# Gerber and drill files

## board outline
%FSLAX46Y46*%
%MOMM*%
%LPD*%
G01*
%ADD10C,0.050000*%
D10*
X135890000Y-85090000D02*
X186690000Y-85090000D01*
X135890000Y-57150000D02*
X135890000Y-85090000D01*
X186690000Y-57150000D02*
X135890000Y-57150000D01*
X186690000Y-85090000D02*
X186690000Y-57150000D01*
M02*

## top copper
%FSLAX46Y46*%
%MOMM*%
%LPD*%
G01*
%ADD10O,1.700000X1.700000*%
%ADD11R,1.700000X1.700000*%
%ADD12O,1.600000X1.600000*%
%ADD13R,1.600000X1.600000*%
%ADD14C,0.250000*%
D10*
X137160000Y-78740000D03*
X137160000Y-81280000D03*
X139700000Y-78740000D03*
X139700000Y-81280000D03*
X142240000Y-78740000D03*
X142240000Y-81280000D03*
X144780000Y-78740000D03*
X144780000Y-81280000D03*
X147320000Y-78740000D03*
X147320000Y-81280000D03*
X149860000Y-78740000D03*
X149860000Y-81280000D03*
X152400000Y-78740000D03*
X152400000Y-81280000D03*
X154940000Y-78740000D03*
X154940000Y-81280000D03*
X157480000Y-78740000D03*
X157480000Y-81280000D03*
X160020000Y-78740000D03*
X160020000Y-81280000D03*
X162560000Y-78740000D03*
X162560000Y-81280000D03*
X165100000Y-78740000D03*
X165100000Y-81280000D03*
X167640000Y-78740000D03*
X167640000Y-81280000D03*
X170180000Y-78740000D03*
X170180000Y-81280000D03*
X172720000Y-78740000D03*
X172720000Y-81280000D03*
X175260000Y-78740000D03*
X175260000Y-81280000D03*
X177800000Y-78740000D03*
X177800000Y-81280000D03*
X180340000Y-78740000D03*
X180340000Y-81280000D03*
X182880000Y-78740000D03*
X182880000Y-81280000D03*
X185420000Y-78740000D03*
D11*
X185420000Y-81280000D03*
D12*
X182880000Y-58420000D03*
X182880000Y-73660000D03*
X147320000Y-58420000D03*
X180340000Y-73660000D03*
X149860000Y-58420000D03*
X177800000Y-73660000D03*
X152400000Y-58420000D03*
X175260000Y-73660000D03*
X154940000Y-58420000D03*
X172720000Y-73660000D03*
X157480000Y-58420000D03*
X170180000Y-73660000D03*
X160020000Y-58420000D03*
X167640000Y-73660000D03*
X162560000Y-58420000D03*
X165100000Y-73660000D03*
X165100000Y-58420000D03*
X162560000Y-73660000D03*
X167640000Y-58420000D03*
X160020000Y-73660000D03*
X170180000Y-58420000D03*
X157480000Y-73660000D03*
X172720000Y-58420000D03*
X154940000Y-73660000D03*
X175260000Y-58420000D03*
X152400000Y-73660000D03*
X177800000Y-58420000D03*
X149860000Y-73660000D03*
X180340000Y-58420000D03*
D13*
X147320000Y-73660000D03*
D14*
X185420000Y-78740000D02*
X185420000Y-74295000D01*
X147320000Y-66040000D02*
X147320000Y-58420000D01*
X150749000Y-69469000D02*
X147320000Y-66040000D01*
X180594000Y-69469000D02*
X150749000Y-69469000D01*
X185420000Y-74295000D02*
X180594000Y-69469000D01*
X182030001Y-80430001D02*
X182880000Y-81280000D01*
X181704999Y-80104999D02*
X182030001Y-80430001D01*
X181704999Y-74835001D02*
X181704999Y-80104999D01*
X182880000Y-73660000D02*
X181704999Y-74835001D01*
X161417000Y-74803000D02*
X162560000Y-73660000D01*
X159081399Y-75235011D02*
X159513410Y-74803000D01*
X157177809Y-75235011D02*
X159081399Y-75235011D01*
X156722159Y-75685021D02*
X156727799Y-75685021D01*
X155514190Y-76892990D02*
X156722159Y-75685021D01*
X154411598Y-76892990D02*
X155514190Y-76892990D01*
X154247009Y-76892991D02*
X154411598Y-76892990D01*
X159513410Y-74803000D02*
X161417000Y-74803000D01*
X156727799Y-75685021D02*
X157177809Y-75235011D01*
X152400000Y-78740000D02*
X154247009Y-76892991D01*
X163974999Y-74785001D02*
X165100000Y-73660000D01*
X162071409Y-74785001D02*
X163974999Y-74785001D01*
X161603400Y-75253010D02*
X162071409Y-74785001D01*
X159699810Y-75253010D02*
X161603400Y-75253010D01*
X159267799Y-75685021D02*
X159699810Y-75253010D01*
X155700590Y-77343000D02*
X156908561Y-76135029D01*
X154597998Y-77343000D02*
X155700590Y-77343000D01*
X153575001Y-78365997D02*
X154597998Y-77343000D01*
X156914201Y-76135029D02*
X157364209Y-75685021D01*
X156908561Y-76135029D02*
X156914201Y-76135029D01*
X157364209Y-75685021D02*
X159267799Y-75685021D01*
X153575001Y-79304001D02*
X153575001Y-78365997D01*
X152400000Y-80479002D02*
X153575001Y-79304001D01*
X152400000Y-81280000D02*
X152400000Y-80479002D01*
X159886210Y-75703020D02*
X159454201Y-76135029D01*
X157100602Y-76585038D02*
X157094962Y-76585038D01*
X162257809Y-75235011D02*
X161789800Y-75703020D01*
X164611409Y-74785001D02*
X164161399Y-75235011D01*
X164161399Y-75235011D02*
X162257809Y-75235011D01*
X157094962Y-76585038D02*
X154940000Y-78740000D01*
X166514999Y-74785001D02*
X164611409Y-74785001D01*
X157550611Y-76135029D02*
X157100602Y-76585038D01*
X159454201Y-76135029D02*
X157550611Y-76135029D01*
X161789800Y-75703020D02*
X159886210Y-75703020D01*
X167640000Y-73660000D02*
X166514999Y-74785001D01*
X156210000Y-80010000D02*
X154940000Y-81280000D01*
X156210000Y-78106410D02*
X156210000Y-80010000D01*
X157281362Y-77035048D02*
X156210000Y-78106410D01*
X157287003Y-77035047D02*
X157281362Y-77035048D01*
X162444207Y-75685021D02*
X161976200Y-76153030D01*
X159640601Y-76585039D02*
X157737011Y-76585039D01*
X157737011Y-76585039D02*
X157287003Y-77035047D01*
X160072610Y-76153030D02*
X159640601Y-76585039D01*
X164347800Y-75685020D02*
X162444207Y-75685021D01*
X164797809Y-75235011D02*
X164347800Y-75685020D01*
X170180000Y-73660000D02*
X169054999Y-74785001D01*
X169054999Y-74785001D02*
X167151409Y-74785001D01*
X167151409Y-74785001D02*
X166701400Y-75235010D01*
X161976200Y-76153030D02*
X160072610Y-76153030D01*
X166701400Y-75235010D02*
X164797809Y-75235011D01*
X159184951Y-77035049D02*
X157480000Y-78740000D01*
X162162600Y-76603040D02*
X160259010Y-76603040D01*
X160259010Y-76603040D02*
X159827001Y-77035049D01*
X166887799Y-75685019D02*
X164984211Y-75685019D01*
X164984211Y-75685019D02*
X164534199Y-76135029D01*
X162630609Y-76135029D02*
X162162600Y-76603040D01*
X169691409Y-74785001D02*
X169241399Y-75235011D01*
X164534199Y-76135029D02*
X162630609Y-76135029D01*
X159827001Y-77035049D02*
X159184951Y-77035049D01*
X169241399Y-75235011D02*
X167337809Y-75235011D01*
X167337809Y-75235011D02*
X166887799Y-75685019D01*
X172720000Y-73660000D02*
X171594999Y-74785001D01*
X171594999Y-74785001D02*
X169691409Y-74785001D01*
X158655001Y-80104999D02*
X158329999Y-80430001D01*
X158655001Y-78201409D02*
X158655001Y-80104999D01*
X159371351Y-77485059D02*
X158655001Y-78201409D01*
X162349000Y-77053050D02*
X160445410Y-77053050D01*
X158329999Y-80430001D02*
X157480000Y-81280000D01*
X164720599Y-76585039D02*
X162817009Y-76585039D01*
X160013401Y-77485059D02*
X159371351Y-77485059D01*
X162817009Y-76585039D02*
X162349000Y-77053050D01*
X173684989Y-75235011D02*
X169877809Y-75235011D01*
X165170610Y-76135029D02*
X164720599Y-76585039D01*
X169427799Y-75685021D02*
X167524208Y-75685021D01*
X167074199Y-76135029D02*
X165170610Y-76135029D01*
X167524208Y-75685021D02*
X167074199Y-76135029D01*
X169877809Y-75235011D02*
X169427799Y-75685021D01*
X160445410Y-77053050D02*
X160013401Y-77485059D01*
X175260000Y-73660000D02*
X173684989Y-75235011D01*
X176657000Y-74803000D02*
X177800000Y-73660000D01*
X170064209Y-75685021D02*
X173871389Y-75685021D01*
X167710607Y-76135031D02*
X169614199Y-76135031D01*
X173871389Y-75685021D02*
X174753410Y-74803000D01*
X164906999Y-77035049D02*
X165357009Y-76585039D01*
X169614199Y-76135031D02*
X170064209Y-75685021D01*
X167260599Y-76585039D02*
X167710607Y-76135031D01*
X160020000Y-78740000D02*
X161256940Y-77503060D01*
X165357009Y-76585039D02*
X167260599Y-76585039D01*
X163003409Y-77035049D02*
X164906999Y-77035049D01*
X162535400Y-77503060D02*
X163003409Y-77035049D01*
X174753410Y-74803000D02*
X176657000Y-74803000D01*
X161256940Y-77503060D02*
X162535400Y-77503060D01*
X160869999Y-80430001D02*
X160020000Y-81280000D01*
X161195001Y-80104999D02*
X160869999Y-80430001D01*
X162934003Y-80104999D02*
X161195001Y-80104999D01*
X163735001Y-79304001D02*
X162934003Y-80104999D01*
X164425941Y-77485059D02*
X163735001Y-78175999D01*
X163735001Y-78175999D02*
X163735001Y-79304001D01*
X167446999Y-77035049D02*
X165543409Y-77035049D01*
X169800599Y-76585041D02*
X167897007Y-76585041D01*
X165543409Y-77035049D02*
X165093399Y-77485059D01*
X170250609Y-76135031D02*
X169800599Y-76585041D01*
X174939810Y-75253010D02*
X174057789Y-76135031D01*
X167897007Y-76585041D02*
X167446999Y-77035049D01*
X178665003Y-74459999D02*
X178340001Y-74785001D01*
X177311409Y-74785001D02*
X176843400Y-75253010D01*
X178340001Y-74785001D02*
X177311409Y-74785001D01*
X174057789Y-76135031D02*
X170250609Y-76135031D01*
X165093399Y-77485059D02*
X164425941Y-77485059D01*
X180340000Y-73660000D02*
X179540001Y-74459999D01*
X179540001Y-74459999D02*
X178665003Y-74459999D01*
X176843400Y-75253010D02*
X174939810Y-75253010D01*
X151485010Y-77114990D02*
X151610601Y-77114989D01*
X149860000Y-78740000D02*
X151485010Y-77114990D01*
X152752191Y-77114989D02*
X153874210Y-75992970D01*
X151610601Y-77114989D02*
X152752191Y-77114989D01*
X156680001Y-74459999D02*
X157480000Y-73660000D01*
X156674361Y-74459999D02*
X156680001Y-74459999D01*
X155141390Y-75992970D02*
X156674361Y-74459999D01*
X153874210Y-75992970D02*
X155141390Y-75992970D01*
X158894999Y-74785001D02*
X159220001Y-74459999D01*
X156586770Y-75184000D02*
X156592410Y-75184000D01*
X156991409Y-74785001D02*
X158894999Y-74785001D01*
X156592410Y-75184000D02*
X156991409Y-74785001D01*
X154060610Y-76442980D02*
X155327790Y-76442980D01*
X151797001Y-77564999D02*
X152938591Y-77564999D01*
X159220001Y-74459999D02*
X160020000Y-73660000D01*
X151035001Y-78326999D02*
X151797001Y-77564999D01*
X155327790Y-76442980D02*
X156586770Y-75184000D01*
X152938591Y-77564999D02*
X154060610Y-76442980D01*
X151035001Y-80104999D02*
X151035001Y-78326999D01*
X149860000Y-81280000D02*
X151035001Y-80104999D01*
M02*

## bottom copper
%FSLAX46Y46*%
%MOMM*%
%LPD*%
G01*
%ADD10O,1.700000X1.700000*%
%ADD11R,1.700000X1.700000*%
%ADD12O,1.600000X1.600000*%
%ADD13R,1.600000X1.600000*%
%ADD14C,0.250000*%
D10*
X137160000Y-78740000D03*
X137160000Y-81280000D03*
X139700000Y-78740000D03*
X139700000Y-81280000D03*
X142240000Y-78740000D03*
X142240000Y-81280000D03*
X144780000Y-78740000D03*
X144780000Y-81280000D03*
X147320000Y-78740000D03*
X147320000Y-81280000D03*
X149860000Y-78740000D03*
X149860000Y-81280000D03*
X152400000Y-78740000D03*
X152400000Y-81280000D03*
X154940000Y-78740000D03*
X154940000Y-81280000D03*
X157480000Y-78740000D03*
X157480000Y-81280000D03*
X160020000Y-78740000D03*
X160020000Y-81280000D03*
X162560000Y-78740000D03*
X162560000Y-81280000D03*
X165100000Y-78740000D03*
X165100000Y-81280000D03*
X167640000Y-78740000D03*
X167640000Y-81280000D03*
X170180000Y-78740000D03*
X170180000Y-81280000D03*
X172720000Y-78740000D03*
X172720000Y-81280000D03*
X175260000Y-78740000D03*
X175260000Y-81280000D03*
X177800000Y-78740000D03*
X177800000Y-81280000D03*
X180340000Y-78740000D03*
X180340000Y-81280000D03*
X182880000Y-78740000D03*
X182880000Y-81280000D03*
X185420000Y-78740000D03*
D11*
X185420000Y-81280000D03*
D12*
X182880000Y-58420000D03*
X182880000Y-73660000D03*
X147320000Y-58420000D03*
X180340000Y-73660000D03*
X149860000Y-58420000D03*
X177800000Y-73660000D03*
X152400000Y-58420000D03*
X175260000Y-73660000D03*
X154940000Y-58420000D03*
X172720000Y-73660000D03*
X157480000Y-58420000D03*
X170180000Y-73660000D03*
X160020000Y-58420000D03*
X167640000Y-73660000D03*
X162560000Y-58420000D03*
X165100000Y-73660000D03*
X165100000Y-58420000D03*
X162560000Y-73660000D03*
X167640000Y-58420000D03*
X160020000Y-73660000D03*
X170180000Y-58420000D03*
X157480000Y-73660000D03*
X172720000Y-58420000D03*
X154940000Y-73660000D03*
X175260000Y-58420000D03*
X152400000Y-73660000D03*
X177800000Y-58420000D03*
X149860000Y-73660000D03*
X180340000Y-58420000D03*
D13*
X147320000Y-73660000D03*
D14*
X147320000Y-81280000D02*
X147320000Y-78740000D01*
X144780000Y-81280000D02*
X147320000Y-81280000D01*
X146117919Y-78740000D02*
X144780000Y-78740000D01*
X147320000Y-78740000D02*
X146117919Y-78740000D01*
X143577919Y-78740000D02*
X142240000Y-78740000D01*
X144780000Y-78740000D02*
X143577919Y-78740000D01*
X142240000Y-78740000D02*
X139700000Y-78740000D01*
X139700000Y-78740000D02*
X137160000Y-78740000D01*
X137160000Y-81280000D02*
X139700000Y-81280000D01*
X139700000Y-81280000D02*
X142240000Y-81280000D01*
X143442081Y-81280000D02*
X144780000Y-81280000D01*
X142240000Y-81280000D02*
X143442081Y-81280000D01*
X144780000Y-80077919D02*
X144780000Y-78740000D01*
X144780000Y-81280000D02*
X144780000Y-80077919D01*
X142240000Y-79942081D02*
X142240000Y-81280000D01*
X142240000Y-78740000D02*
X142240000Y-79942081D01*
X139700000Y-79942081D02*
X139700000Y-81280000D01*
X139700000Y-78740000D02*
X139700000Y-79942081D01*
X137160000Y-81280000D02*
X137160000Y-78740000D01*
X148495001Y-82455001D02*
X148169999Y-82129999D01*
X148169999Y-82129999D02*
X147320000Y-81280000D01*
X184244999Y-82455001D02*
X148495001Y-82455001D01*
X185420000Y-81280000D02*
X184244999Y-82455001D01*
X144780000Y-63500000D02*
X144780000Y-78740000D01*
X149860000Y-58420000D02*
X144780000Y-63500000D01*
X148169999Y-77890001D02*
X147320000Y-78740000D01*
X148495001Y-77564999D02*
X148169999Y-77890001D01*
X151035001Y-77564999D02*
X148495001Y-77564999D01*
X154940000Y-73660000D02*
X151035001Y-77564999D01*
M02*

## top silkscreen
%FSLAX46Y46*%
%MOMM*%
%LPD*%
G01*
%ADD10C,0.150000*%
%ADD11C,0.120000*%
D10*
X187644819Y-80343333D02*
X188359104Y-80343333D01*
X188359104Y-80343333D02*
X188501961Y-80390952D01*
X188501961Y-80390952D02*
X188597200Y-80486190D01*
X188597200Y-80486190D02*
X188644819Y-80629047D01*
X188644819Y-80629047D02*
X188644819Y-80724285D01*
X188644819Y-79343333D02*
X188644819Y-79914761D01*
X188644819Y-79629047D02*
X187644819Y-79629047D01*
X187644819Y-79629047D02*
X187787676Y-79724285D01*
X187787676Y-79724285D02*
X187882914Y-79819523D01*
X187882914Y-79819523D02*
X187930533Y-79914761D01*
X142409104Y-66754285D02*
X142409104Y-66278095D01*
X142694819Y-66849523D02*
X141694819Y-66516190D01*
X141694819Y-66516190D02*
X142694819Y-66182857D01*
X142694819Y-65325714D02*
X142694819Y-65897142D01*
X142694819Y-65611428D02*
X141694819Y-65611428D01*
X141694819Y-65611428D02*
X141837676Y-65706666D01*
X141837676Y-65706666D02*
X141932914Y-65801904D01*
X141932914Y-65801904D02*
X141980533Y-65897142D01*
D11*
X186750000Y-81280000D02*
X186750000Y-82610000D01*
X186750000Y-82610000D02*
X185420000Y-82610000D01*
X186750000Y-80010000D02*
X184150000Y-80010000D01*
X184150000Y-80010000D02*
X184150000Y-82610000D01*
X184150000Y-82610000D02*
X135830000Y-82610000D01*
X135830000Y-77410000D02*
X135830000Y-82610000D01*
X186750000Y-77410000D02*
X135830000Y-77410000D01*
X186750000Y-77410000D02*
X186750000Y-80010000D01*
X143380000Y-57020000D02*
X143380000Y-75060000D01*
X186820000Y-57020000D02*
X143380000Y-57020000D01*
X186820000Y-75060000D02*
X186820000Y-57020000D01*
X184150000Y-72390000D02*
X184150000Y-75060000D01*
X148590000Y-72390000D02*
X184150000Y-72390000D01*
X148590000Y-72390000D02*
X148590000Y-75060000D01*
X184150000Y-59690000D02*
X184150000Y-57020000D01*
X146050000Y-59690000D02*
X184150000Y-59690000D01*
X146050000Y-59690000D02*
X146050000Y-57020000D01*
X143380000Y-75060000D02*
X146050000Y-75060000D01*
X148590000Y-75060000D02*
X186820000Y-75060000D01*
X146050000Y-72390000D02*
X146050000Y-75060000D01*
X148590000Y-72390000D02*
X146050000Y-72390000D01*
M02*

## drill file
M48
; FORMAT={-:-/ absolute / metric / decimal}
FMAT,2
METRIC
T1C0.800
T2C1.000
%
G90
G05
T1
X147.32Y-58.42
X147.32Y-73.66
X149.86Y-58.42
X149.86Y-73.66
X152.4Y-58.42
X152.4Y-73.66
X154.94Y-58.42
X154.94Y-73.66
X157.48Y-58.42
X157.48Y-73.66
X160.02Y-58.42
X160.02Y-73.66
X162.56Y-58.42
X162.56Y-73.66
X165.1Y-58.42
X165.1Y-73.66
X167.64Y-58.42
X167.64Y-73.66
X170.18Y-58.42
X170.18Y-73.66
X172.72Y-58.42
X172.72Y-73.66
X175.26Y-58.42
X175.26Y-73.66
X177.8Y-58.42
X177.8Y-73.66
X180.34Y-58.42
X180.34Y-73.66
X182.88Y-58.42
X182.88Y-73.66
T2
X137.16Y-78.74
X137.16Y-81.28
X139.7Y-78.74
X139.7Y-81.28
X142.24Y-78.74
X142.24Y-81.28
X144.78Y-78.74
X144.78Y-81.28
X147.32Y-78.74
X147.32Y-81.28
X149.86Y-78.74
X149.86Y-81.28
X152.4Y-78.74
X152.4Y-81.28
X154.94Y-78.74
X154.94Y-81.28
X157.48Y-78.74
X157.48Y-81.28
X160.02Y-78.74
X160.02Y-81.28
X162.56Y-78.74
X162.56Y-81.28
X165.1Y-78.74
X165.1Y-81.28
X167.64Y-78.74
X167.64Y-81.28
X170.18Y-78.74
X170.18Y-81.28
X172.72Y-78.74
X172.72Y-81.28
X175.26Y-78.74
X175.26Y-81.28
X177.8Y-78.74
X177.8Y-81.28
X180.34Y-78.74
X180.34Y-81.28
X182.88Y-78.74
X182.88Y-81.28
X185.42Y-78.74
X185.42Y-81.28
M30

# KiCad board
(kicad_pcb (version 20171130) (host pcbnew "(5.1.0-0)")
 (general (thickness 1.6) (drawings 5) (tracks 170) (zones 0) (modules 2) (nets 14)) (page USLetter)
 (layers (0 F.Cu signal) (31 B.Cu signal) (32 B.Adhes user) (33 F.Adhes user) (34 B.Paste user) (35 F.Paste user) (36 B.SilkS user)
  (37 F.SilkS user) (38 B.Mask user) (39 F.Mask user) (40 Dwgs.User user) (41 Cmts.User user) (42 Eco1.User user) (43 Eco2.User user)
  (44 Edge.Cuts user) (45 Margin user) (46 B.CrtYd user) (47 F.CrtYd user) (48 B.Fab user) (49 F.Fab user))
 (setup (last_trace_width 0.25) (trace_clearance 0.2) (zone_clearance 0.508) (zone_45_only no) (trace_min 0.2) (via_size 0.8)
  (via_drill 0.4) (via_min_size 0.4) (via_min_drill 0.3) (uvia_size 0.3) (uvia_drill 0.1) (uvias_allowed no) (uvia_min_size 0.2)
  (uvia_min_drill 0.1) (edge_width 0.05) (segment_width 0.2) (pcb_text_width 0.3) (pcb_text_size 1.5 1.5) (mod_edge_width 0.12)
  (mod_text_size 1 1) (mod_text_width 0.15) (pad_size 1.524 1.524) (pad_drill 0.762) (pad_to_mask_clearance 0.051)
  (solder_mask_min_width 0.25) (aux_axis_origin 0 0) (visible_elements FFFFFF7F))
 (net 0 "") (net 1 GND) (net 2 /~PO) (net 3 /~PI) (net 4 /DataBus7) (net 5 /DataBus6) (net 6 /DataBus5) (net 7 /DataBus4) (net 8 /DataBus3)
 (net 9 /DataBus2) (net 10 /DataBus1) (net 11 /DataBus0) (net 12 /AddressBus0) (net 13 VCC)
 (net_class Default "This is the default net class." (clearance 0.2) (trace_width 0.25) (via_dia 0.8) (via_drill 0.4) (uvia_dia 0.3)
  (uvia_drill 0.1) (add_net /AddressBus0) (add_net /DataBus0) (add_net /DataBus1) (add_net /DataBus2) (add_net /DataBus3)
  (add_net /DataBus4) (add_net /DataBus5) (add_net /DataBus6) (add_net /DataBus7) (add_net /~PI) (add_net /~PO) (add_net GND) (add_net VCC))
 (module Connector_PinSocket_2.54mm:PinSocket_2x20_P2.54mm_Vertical (layer F.Cu) (at 185.42 81.28 270)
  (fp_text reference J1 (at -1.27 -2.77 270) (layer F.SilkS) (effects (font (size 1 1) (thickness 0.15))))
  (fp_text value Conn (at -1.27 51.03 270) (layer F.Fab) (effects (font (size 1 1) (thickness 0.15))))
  (fp_line (start 0 -1.33) (end 1.33 -1.33) (layer F.SilkS) (width 0.12))
  (fp_line (start 1.33 -1.33) (end 1.33 0) (layer F.SilkS) (width 0.12))
  (fp_line (start -1.27 -1.33) (end -1.27 1.27) (layer F.SilkS) (width 0.12))
  (fp_line (start -1.27 1.27) (end 1.33 1.27) (layer F.SilkS) (width 0.12))
  (fp_line (start 1.33 1.27) (end 1.33 49.59) (layer F.SilkS) (width 0.12))
  (fp_line (start -3.87 49.59) (end 1.33 49.59) (layer F.SilkS) (width 0.12))
  (fp_line (start -3.87 -1.33) (end -3.87 49.59) (layer F.SilkS) (width 0.12))
  (fp_line (start -3.87 -1.33) (end -1.27 -1.33) (layer F.SilkS) (width 0.12))
  (pad 40 thru_hole oval (at -2.54 48.26 270) (size 1.7 1.7) (drill 1) (layers *.Cu *.Mask) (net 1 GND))
  (pad 39 thru_hole oval (at 0 48.26 270) (size 1.7 1.7) (drill 1) (layers *.Cu *.Mask) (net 1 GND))
  (pad 38 thru_hole oval (at -2.54 45.72 270) (size 1.7 1.7) (drill 1) (layers *.Cu *.Mask) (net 1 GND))
  (pad 37 thru_hole oval (at 0 45.72 270) (size 1.7 1.7) (drill 1) (layers *.Cu *.Mask) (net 1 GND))
  (pad 36 thru_hole oval (at -2.54 43.18 270) (size 1.7 1.7) (drill 1) (layers *.Cu *.Mask) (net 1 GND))
  (pad 35 thru_hole oval (at 0 43.18 270) (size 1.7 1.7) (drill 1) (layers *.Cu *.Mask) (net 1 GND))
  (pad 34 thru_hole oval (at -2.54 40.64 270) (size 1.7 1.7) (drill 1) (layers *.Cu *.Mask) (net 1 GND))
  (pad 33 thru_hole oval (at 0 40.64 270) (size 1.7 1.7) (drill 1) (layers *.Cu *.Mask) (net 1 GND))
  (pad 32 thru_hole oval (at -2.54 38.1 270) (size 1.7 1.7) (drill 1) (layers *.Cu *.Mask) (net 1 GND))
  (pad 31 thru_hole oval (at 0 38.1 270) (size 1.7 1.7) (drill 1) (layers *.Cu *.Mask) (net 1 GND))
  (pad 30 thru_hole oval (at -2.54 35.56 270) (size 1.7 1.7) (drill 1) (layers *.Cu *.Mask) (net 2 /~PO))
  (pad 29 thru_hole oval (at 0 35.56 270) (size 1.7 1.7) (drill 1) (layers *.Cu *.Mask) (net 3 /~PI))
  (pad 28 thru_hole oval (at -2.54 33.02 270) (size 1.7 1.7) (drill 1) (layers *.Cu *.Mask) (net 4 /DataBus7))
  (pad 27 thru_hole oval (at 0 33.02 270) (size 1.7 1.7) (drill 1) (layers *.Cu *.Mask) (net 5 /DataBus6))
  (pad 26 thru_hole oval (at -2.54 30.48 270) (size 1.7 1.7) (drill 1) (layers *.Cu *.Mask) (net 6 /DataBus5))
  (pad 25 thru_hole oval (at 0 30.48 270) (size 1.7 1.7) (drill 1) (layers *.Cu *.Mask) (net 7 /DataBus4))
  (pad 24 thru_hole oval (at -2.54 27.94 270) (size 1.7 1.7) (drill 1) (layers *.Cu *.Mask) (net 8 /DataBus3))
  (pad 23 thru_hole oval (at 0 27.94 270) (size 1.7 1.7) (drill 1) (layers *.Cu *.Mask) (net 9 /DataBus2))
  (pad 22 thru_hole oval (at -2.54 25.4 270) (size 1.7 1.7) (drill 1) (layers *.Cu *.Mask) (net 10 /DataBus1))
  (pad 21 thru_hole oval (at 0 25.4 270) (size 1.7 1.7) (drill 1) (layers *.Cu *.Mask) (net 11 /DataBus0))
  (pad 20 thru_hole oval (at -2.54 22.86 270) (size 1.7 1.7) (drill 1) (layers *.Cu *.Mask))
  (pad 19 thru_hole oval (at 0 22.86 270) (size 1.7 1.7) (drill 1) (layers *.Cu *.Mask))
  (pad 18 thru_hole oval (at -2.54 20.32 270) (size 1.7 1.7) (drill 1) (layers *.Cu *.Mask))
  (pad 17 thru_hole oval (at 0 20.32 270) (size 1.7 1.7) (drill 1) (layers *.Cu *.Mask))
  (pad 16 thru_hole oval (at -2.54 17.78 270) (size 1.7 1.7) (drill 1) (layers *.Cu *.Mask))
  (pad 15 thru_hole oval (at 0 17.78 270) (size 1.7 1.7) (drill 1) (layers *.Cu *.Mask))
  (pad 14 thru_hole oval (at -2.54 15.24 270) (size 1.7 1.7) (drill 1) (layers *.Cu *.Mask))
  (pad 13 thru_hole oval (at 0 15.24 270) (size 1.7 1.7) (drill 1) (layers *.Cu *.Mask))
  (pad 12 thru_hole oval (at -2.54 12.7 270) (size 1.7 1.7) (drill 1) (layers *.Cu *.Mask))
  (pad 11 thru_hole oval (at 0 12.7 270) (size 1.7 1.7) (drill 1) (layers *.Cu *.Mask))
  (pad 10 thru_hole oval (at -2.54 10.16 270) (size 1.7 1.7) (drill 1) (layers *.Cu *.Mask))
  (pad 9 thru_hole oval (at 0 10.16 270) (size 1.7 1.7) (drill 1) (layers *.Cu *.Mask))
  (pad 8 thru_hole oval (at -2.54 7.62 270) (size 1.7 1.7) (drill 1) (layers *.Cu *.Mask))
  (pad 7 thru_hole oval (at 0 7.62 270) (size 1.7 1.7) (drill 1) (layers *.Cu *.Mask))
  (pad 6 thru_hole oval (at -2.54 5.08 270) (size 1.7 1.7) (drill 1) (layers *.Cu *.Mask))
  (pad 5 thru_hole oval (at 0 5.08 270) (size 1.7 1.7) (drill 1) (layers *.Cu *.Mask))
  (pad 4 thru_hole oval (at -2.54 2.54 270) (size 1.7 1.7) (drill 1) (layers *.Cu *.Mask))
  (pad 3 thru_hole oval (at 0 2.54 270) (size 1.7 1.7) (drill 1) (layers *.Cu *.Mask) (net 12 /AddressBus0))
  (pad 2 thru_hole oval (at -2.54 0 270) (size 1.7 1.7) (drill 1) (layers *.Cu *.Mask) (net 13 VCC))
  (pad 1 thru_hole rect (at 0 0 270) (size 1.7 1.7) (drill 1) (layers *.Cu *.Mask) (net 1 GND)))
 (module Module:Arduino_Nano (layer F.Cu) (at 147.32 73.66 90)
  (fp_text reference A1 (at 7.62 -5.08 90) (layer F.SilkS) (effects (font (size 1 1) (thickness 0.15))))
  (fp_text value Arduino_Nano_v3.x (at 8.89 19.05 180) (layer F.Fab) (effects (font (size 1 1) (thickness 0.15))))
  (fp_line (start 16.64 -3.94) (end -1.4 -3.94) (layer F.SilkS) (width 0.12))
  (fp_line (start 16.64 39.5) (end 16.64 -3.94) (layer F.SilkS) (width 0.12))
  (fp_line (start -1.4 39.5) (end 16.64 39.5) (layer F.SilkS) (width 0.12))
  (fp_line (start 1.27 36.83) (end -1.4 36.83) (layer F.SilkS) (width 0.12))
  (fp_line (start 1.27 1.27) (end 1.27 36.83) (layer F.SilkS) (width 0.12))
  (fp_line (start 1.27 1.27) (end -1.4 1.27) (layer F.SilkS) (width 0.12))
  (fp_line (start 13.97 36.83) (end 16.64 36.83) (layer F.SilkS) (width 0.12))
  (fp_line (start 13.97 -1.27) (end 13.97 36.83) (layer F.SilkS) (width 0.12))
  (fp_line (start 13.97 -1.27) (end 16.64 -1.27) (layer F.SilkS) (width 0.12))
  (fp_line (start -1.4 -3.94) (end -1.4 -1.27) (layer F.SilkS) (width 0.12))
  (fp_line (start -1.4 1.27) (end -1.4 39.5) (layer F.SilkS) (width 0.12))
  (fp_line (start 1.27 -1.27) (end -1.4 -1.27) (layer F.SilkS) (width 0.12))
  (fp_line (start 1.27 1.27) (end 1.27 -1.27) (layer F.SilkS) (width 0.12))
  (pad 16 thru_hole oval (at 15.24 35.56 90) (size 1.6 1.6) (drill 0.8) (layers *.Cu *.Mask))
  (pad 15 thru_hole oval (at 0 35.56 90) (size 1.6 1.6) (drill 0.8) (layers *.Cu *.Mask) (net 12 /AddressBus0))
  (pad 30 thru_hole oval (at 15.24 0 90) (size 1.6 1.6) (drill 0.8) (layers *.Cu *.Mask) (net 13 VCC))
  (pad 14 thru_hole oval (at 0 33.02 90) (size 1.6 1.6) (drill 0.8) (layers *.Cu *.Mask) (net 11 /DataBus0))
  (pad 29 thru_hole oval (at 15.24 2.54 90) (size 1.6 1.6) (drill 0.8) (layers *.Cu *.Mask) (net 1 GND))
  (pad 13 thru_hole oval (at 0 30.48 90) (size 1.6 1.6) (drill 0.8) (layers *.Cu *.Mask) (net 10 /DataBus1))
  (pad 28 thru_hole oval (at 15.24 5.08 90) (size 1.6 1.6) (drill 0.8) (layers *.Cu *.Mask))
  (pad 12 thru_hole oval (at 0 27.94 90) (size 1.6 1.6) (drill 0.8) (layers *.Cu *.Mask) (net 9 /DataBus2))
  (pad 27 thru_hole oval (at 15.24 7.62 90) (size 1.6 1.6) (drill 0.8) (layers *.Cu *.Mask))
  (pad 11 thru_hole oval (at 0 25.4 90) (size 1.6 1.6) (drill 0.8) (layers *.Cu *.Mask) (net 8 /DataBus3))
  (pad 26 thru_hole oval (at 15.24 10.16 90) (size 1.6 1.6) (drill 0.8) (layers *.Cu *.Mask))
  (pad 10 thru_hole oval (at 0 22.86 90) (size 1.6 1.6) (drill 0.8) (layers *.Cu *.Mask) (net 7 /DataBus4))
  (pad 25 thru_hole oval (at 15.24 12.7 90) (size 1.6 1.6) (drill 0.8) (layers *.Cu *.Mask))
  (pad 9 thru_hole oval (at 0 20.32 90) (size 1.6 1.6) (drill 0.8) (layers *.Cu *.Mask) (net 6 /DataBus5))
  (pad 24 thru_hole oval (at 15.24 15.24 90) (size 1.6 1.6) (drill 0.8) (layers *.Cu *.Mask))
  (pad 8 thru_hole oval (at 0 17.78 90) (size 1.6 1.6) (drill 0.8) (layers *.Cu *.Mask) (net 5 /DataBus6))
  (pad 23 thru_hole oval (at 15.24 17.78 90) (size 1.6 1.6) (drill 0.8) (layers *.Cu *.Mask))
  (pad 7 thru_hole oval (at 0 15.24 90) (size 1.6 1.6) (drill 0.8) (layers *.Cu *.Mask) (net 4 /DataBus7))
  (pad 22 thru_hole oval (at 15.24 20.32 90) (size 1.6 1.6) (drill 0.8) (layers *.Cu *.Mask))
  (pad 6 thru_hole oval (at 0 12.7 90) (size 1.6 1.6) (drill 0.8) (layers *.Cu *.Mask) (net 3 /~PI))
  (pad 21 thru_hole oval (at 15.24 22.86 90) (size 1.6 1.6) (drill 0.8) (layers *.Cu *.Mask))
  (pad 5 thru_hole oval (at 0 10.16 90) (size 1.6 1.6) (drill 0.8) (layers *.Cu *.Mask) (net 2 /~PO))
  (pad 20 thru_hole oval (at 15.24 25.4 90) (size 1.6 1.6) (drill 0.8) (layers *.Cu *.Mask))
  (pad 4 thru_hole oval (at 0 7.62 90) (size 1.6 1.6) (drill 0.8) (layers *.Cu *.Mask) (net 1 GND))
  (pad 19 thru_hole oval (at 15.24 27.94 90) (size 1.6 1.6) (drill 0.8) (layers *.Cu *.Mask))
  (pad 3 thru_hole oval (at 0 5.08 90) (size 1.6 1.6) (drill 0.8) (layers *.Cu *.Mask))
  (pad 18 thru_hole oval (at 15.24 30.48 90) (size 1.6 1.6) (drill 0.8) (layers *.Cu *.Mask))
  (pad 2 thru_hole oval (at 0 2.54 90) (size 1.6 1.6) (drill 0.8) (layers *.Cu *.Mask))
  (pad 17 thru_hole oval (at 15.24 33.02 90) (size 1.6 1.6) (drill 0.8) (layers *.Cu *.Mask))
  (pad 1 thru_hole rect (at 0 0 90) (size 1.6 1.6) (drill 0.8) (layers *.Cu *.Mask)))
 (gr_line (start 135.89 85.09) (end 186.69 85.09) (layer Edge.Cuts) (width 0.05))
 (gr_line (start 135.89 57.15) (end 135.89 85.09) (layer Edge.Cuts) (width 0.05))
 (gr_line (start 186.69 57.15) (end 135.89 57.15) (layer Edge.Cuts) (width 0.05))
 (gr_line (start 186.69 85.09) (end 186.69 57.15) (layer Edge.Cuts) (width 0.05))
 (segment (start 185.42 78.74) (end 185.42 74.295) (width 0.25) (layer F.Cu) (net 13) (status 1000000))
 (segment (start 147.32 66.04) (end 147.32 58.42) (width 0.25) (layer F.Cu) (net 13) (status 1000000))
 (segment (start 150.749 69.469) (end 147.32 66.04) (width 0.25) (layer F.Cu) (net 13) (status 1000000))
 (segment (start 180.594 69.469) (end 150.749 69.469) (width 0.25) (layer F.Cu) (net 13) (status 1000000))
 (segment (start 185.42 74.295) (end 180.594 69.469) (width 0.25) (layer F.Cu) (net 13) (status 1000000))
 (segment (start 147.32 81.28) (end 147.32 78.74) (width 0.25) (layer B.Cu) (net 1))
 (segment (start 144.78 81.28) (end 147.32 81.28) (width 0.25) (layer B.Cu) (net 1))
 (segment (start 146.117919 78.74) (end 144.78 78.74) (width 0.25) (layer B.Cu) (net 1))
 (segment (start 147.32 78.74) (end 146.117919 78.74) (width 0.25) (layer B.Cu) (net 1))
 (segment (start 143.577919 78.74) (end 142.24 78.74) (width 0.25) (layer B.Cu) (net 1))
 (segment (start 144.78 78.74) (end 143.577919 78.74) (width 0.25) (layer B.Cu) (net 1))
 (segment (start 142.24 78.74) (end 139.7 78.74) (width 0.25) (layer B.Cu) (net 1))
 (segment (start 139.7 78.74) (end 137.16 78.74) (width 0.25) (layer B.Cu) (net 1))
 (segment (start 137.16 81.28) (end 139.7 81.28) (width 0.25) (layer B.Cu) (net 1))
 (segment (start 139.7 81.28) (end 142.24 81.28) (width 0.25) (layer B.Cu) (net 1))
 (segment (start 143.442081 81.28) (end 144.78 81.28) (width 0.25) (layer B.Cu) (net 1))
 (segment (start 142.24 81.28) (end 143.442081 81.28) (width 0.25) (layer B.Cu) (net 1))
 (segment (start 144.78 80.077919) (end 144.78 78.74) (width 0.25) (layer B.Cu) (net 1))
 (segment (start 144.78 81.28) (end 144.78 80.077919) (width 0.25) (layer B.Cu) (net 1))
 (segment (start 142.24 79.942081) (end 142.24 81.28) (width 0.25) (layer B.Cu) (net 1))
 (segment (start 142.24 78.74) (end 142.24 79.942081) (width 0.25) (layer B.Cu) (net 1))
 (segment (start 139.7 79.942081) (end 139.7 81.28) (width 0.25) (layer B.Cu) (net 1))
 (segment (start 139.7 78.74) (end 139.7 79.942081) (width 0.25) (layer B.Cu) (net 1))
 (segment (start 137.16 81.28) (end 137.16 78.74) (width 0.25) (layer B.Cu) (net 1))
 (segment (start 148.495001 82.455001) (end 148.169999 82.129999) (width 0.25) (layer B.Cu) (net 1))
 (segment (start 148.169999 82.129999) (end 147.32 81.28) (width 0.25) (layer B.Cu) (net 1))
 (segment (start 184.244999 82.455001) (end 148.495001 82.455001) (width 0.25) (layer B.Cu) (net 1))
 (segment (start 185.42 81.28) (end 184.244999 82.455001) (width 0.25) (layer B.Cu) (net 1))
 (segment (start 144.78 63.5) (end 144.78 78.74) (width 0.25) (layer B.Cu) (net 1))
 (segment (start 149.86 58.42) (end 144.78 63.5) (width 0.25) (layer B.Cu) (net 1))
 (segment (start 148.169999 77.890001) (end 147.32 78.74) (width 0.25) (layer B.Cu) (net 1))
 (segment (start 148.495001 77.564999) (end 148.169999 77.890001) (width 0.25) (layer B.Cu) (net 1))
 (segment (start 151.035001 77.564999) (end 148.495001 77.564999) (width 0.25) (layer B.Cu) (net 1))
 (segment (start 154.94 73.66) (end 151.035001 77.564999) (width 0.25) (layer B.Cu) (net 1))
 (segment (start 182.030001 80.430001) (end 182.88 81.28) (width 0.25) (layer F.Cu) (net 12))
 (segment (start 181.704999 80.104999) (end 182.030001 80.430001) (width 0.25) (layer F.Cu) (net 12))
 (segment (start 181.704999 74.835001) (end 181.704999 80.104999) (width 0.25) (layer F.Cu) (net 12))
 (segment (start 182.88 73.66) (end 181.704999 74.835001) (width 0.25) (layer F.Cu) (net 12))
 (segment (start 161.417 74.803) (end 162.56 73.66) (width 0.25) (layer F.Cu) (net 4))
 (segment (start 159.081399 75.235011) (end 159.51341 74.803) (width 0.25) (layer F.Cu) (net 4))
 (segment (start 157.177809 75.235011) (end 159.081399 75.235011) (width 0.25) (layer F.Cu) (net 4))
 (segment (start 156.722159 75.685021) (end 156.727799 75.685021) (width 0.25) (layer F.Cu) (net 4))
 (segment (start 155.51419 76.89299) (end 156.722159 75.685021) (width 0.25) (layer F.Cu) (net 4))
 (segment (start 154.411598 76.89299) (end 155.51419 76.89299) (width 0.25) (layer F.Cu) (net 4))
 (segment (start 154.247009 76.892991) (end 154.411598 76.89299) (width 0.25) (layer F.Cu) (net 4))
 (segment (start 159.51341 74.803) (end 161.417 74.803) (width 0.25) (layer F.Cu) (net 4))
 (segment (start 156.727799 75.685021) (end 157.177809 75.235011) (width 0.25) (layer F.Cu) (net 4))
 (segment (start 152.4 78.74) (end 154.247009 76.892991) (width 0.25) (layer F.Cu) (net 4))
 (segment (start 163.974999 74.785001) (end 165.1 73.66) (width 0.25) (layer F.Cu) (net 5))
 (segment (start 162.071409 74.785001) (end 163.974999 74.785001) (width 0.25) (layer F.Cu) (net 5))
 (segment (start 161.6034 75.25301) (end 162.071409 74.785001) (width 0.25) (layer F.Cu) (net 5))
 (segment (start 159.69981 75.25301) (end 161.6034 75.25301) (width 0.25) (layer F.Cu) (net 5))
 (segment (start 159.267799 75.685021) (end 159.69981 75.25301) (width 0.25) (layer F.Cu) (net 5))
 (segment (start 155.70059 77.343) (end 156.908561 76.135029) (width 0.25) (layer F.Cu) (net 5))
 (segment (start 154.597998 77.343) (end 155.70059 77.343) (width 0.25) (layer F.Cu) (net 5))
 (segment (start 153.575001 78.365997) (end 154.597998 77.343) (width 0.25) (layer F.Cu) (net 5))
 (segment (start 156.914201 76.135029) (end 157.364209 75.685021) (width 0.25) (layer F.Cu) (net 5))
 (segment (start 156.908561 76.135029) (end 156.914201 76.135029) (width 0.25) (layer F.Cu) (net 5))
 (segment (start 157.364209 75.685021) (end 159.267799 75.685021) (width 0.25) (layer F.Cu) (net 5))
 (segment (start 153.575001 79.304001) (end 153.575001 78.365997) (width 0.25) (layer F.Cu) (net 5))
 (segment (start 152.4 80.479002) (end 153.575001 79.304001) (width 0.25) (layer F.Cu) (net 5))
 (segment (start 152.4 81.28) (end 152.4 80.479002) (width 0.25) (layer F.Cu) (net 5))
 (segment (start 159.88621 75.70302) (end 159.454201 76.135029) (width 0.25) (layer F.Cu) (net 6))
 (segment (start 157.100602 76.585038) (end 157.094962 76.585038) (width 0.25) (layer F.Cu) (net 6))
 (segment (start 162.257809 75.235011) (end 161.7898 75.70302) (width 0.25) (layer F.Cu) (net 6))
 (segment (start 164.611409 74.785001) (end 164.161399 75.235011) (width 0.25) (layer F.Cu) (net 6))
 (segment (start 164.161399 75.235011) (end 162.257809 75.235011) (width 0.25) (layer F.Cu) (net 6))
 (segment (start 157.094962 76.585038) (end 154.94 78.74) (width 0.25) (layer F.Cu) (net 6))
 (segment (start 166.514999 74.785001) (end 164.611409 74.785001) (width 0.25) (layer F.Cu) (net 6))
 (segment (start 157.550611 76.135029) (end 157.100602 76.585038) (width 0.25) (layer F.Cu) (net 6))
 (segment (start 159.454201 76.135029) (end 157.550611 76.135029) (width 0.25) (layer F.Cu) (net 6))
 (segment (start 161.7898 75.70302) (end 159.88621 75.70302) (width 0.25) (layer F.Cu) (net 6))
 (segment (start 167.64 73.66) (end 166.514999 74.785001) (width 0.25) (layer F.Cu) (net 6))
 (segment (start 156.21 80.01) (end 154.94 81.28) (width 0.25) (layer F.Cu) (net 7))
 (segment (start 156.21 78.10641) (end 156.21 80.01) (width 0.25) (layer F.Cu) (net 7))
 (segment (start 157.281362 77.035048) (end 156.21 78.10641) (width 0.25) (layer F.Cu) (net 7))
 (segment (start 157.287003 77.035047) (end 157.281362 77.035048) (width 0.25) (layer F.Cu) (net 7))
 (segment (start 162.444207 75.685021) (end 161.9762 76.15303) (width 0.25) (layer F.Cu) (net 7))
 (segment (start 159.640601 76.585039) (end 157.737011 76.585039) (width 0.25) (layer F.Cu) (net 7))
 (segment (start 157.737011 76.585039) (end 157.287003 77.035047) (width 0.25) (layer F.Cu) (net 7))
 (segment (start 160.07261 76.15303) (end 159.640601 76.585039) (width 0.25) (layer F.Cu) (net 7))
 (segment (start 164.3478 75.68502) (end 162.444207 75.685021) (width 0.25) (layer F.Cu) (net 7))
 (segment (start 164.797809 75.235011) (end 164.3478 75.68502) (width 0.25) (layer F.Cu) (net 7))
 (segment (start 170.18 73.66) (end 169.054999 74.785001) (width 0.25) (layer F.Cu) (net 7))
 (segment (start 169.054999 74.785001) (end 167.151409 74.785001) (width 0.25) (layer F.Cu) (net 7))
 (segment (start 167.151409 74.785001) (end 166.7014 75.23501) (width 0.25) (layer F.Cu) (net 7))
 (segment (start 161.9762 76.15303) (end 160.07261 76.15303) (width 0.25) (layer F.Cu) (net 7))
 (segment (start 166.7014 75.23501) (end 164.797809 75.235011) (width 0.25) (layer F.Cu) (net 7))
 (segment (start 159.184951 77.035049) (end 157.48 78.74) (width 0.25) (layer F.Cu) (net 8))
 (segment (start 162.1626 76.60304) (end 160.25901 76.60304) (width 0.25) (layer F.Cu) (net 8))
 (segment (start 160.25901 76.60304) (end 159.827001 77.035049) (width 0.25) (layer F.Cu) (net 8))
 (segment (start 166.887799 75.685019) (end 164.984211 75.685019) (width 0.25) (layer F.Cu) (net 8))
 (segment (start 164.984211 75.685019) (end 164.534199 76.135029) (width 0.25) (layer F.Cu) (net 8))
 (segment (start 162.630609 76.135029) (end 162.1626 76.60304) (width 0.25) (layer F.Cu) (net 8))
 (segment (start 169.691409 74.785001) (end 169.241399 75.235011) (width 0.25) (layer F.Cu) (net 8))
 (segment (start 164.534199 76.135029) (end 162.630609 76.135029) (width 0.25) (layer F.Cu) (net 8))
 (segment (start 159.827001 77.035049) (end 159.184951 77.035049) (width 0.25) (layer F.Cu) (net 8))
 (segment (start 169.241399 75.235011) (end 167.337809 75.235011) (width 0.25) (layer F.Cu) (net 8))
 (segment (start 167.337809 75.235011) (end 166.887799 75.685019) (width 0.25) (layer F.Cu) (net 8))
 (segment (start 172.72 73.66) (end 171.594999 74.785001) (width 0.25) (layer F.Cu) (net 8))
 (segment (start 171.594999 74.785001) (end 169.691409 74.785001) (width 0.25) (layer F.Cu) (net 8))
 (segment (start 158.655001 80.104999) (end 158.329999 80.430001) (width 0.25) (layer F.Cu) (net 9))
 (segment (start 158.655001 78.201409) (end 158.655001 80.104999) (width 0.25) (layer F.Cu) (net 9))
 (segment (start 159.371351 77.485059) (end 158.655001 78.201409) (width 0.25) (layer F.Cu) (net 9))
 (segment (start 162.349 77.05305) (end 160.44541 77.05305) (width 0.25) (layer F.Cu) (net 9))
 (segment (start 158.329999 80.430001) (end 157.48 81.28) (width 0.25) (layer F.Cu) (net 9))
 (segment (start 164.720599 76.585039) (end 162.817009 76.585039) (width 0.25) (layer F.Cu) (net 9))
 (segment (start 160.013401 77.485059) (end 159.371351 77.485059) (width 0.25) (layer F.Cu) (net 9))
 (segment (start 162.817009 76.585039) (end 162.349 77.05305) (width 0.25) (layer F.Cu) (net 9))
 (segment (start 173.684989 75.235011) (end 169.877809 75.235011) (width 0.25) (layer F.Cu) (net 9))
 (segment (start 165.17061 76.135029) (end 164.720599 76.585039) (width 0.25) (layer F.Cu) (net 9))
 (segment (start 169.427799 75.685021) (end 167.524208 75.685021) (width 0.25) (layer F.Cu) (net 9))
 (segment (start 167.074199 76.135029) (end 165.17061 76.135029) (width 0.25) (layer F.Cu) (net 9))
 (segment (start 167.524208 75.685021) (end 167.074199 76.135029) (width 0.25) (layer F.Cu) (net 9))
 (segment (start 169.877809 75.235011) (end 169.427799 75.685021) (width 0.25) (layer F.Cu) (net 9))
 (segment (start 160.44541 77.05305) (end 160.013401 77.485059) (width 0.25) (layer F.Cu) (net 9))
 (segment (start 175.26 73.66) (end 173.684989 75.235011) (width 0.25) (layer F.Cu) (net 9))
 (segment (start 176.657 74.803) (end 177.8 73.66) (width 0.25) (layer F.Cu) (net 10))
 (segment (start 170.064209 75.685021) (end 173.871389 75.685021) (width 0.25) (layer F.Cu) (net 10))
 (segment (start 167.710607 76.135031) (end 169.614199 76.135031) (width 0.25) (layer F.Cu) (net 10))
 (segment (start 173.871389 75.685021) (end 174.75341 74.803) (width 0.25) (layer F.Cu) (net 10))
 (segment (start 164.906999 77.035049) (end 165.357009 76.585039) (width 0.25) (layer F.Cu) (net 10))
 (segment (start 169.614199 76.135031) (end 170.064209 75.685021) (width 0.25) (layer F.Cu) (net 10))
 (segment (start 167.260599 76.585039) (end 167.710607 76.135031) (width 0.25) (layer F.Cu) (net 10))
 (segment (start 160.02 78.74) (end 161.25694 77.50306) (width 0.25) (layer F.Cu) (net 10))
 (segment (start 165.357009 76.585039) (end 167.260599 76.585039) (width 0.25) (layer F.Cu) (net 10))
 (segment (start 163.003409 77.035049) (end 164.906999 77.035049) (width 0.25) (layer F.Cu) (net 10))
 (segment (start 162.5354 77.50306) (end 163.003409 77.035049) (width 0.25) (layer F.Cu) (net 10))
 (segment (start 174.75341 74.803) (end 176.657 74.803) (width 0.25) (layer F.Cu) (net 10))
 (segment (start 161.25694 77.50306) (end 162.5354 77.50306) (width 0.25) (layer F.Cu) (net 10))
 (segment (start 160.869999 80.430001) (end 160.02 81.28) (width 0.25) (layer F.Cu) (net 11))
 (segment (start 161.195001 80.104999) (end 160.869999 80.430001) (width 0.25) (layer F.Cu) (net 11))
 (segment (start 162.934003 80.104999) (end 161.195001 80.104999) (width 0.25) (layer F.Cu) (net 11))
 (segment (start 163.735001 79.304001) (end 162.934003 80.104999) (width 0.25) (layer F.Cu) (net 11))
 (segment (start 164.425941 77.485059) (end 163.735001 78.175999) (width 0.25) (layer F.Cu) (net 11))
 (segment (start 163.735001 78.175999) (end 163.735001 79.304001) (width 0.25) (layer F.Cu) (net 11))
 (segment (start 167.446999 77.035049) (end 165.543409 77.035049) (width 0.25) (layer F.Cu) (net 11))
 (segment (start 169.800599 76.585041) (end 167.897007 76.585041) (width 0.25) (layer F.Cu) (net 11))
 (segment (start 165.543409 77.035049) (end 165.093399 77.485059) (width 0.25) (layer F.Cu) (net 11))
 (segment (start 170.250609 76.135031) (end 169.800599 76.585041) (width 0.25) (layer F.Cu) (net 11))
 (segment (start 174.93981 75.25301) (end 174.057789 76.135031) (width 0.25) (layer F.Cu) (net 11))
 (segment (start 167.897007 76.585041) (end 167.446999 77.035049) (width 0.25) (layer F.Cu) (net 11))
 (segment (start 178.665003 74.459999) (end 178.340001 74.785001) (width 0.25) (layer F.Cu) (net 11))
 (segment (start 177.311409 74.785001) (end 176.8434 75.25301) (width 0.25) (layer F.Cu) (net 11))
 (segment (start 178.340001 74.785001) (end 177.311409 74.785001) (width 0.25) (layer F.Cu) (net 11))
 (segment (start 174.057789 76.135031) (end 170.250609 76.135031) (width 0.25) (layer F.Cu) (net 11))
 (segment (start 165.093399 77.485059) (end 164.425941 77.485059) (width 0.25) (layer F.Cu) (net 11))
 (segment (start 180.34 73.66) (end 179.540001 74.459999) (width 0.25) (layer F.Cu) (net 11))
 (segment (start 179.540001 74.459999) (end 178.665003 74.459999) (width 0.25) (layer F.Cu) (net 11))
 (segment (start 176.8434 75.25301) (end 174.93981 75.25301) (width 0.25) (layer F.Cu) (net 11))
 (segment (start 151.48501 77.11499) (end 151.610601 77.114989) (width 0.25) (layer F.Cu) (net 2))
 (segment (start 149.86 78.74) (end 151.48501 77.11499) (width 0.25) (layer F.Cu) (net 2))
 (segment (start 152.752191 77.114989) (end 153.87421 75.99297) (width 0.25) (layer F.Cu) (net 2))
 (segment (start 151.610601 77.114989) (end 152.752191 77.114989) (width 0.25) (layer F.Cu) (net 2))
 (segment (start 156.680001 74.459999) (end 157.48 73.66) (width 0.25) (layer F.Cu) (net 2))
 (segment (start 156.674361 74.459999) (end 156.680001 74.459999) (width 0.25) (layer F.Cu) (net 2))
 (segment (start 155.14139 75.99297) (end 156.674361 74.459999) (width 0.25) (layer F.Cu) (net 2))
 (segment (start 153.87421 75.99297) (end 155.14139 75.99297) (width 0.25) (layer F.Cu) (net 2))
 (segment (start 158.894999 74.785001) (end 159.220001 74.459999) (width 0.25) (layer F.Cu) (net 3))
 (segment (start 156.58677 75.184) (end 156.59241 75.184) (width 0.25) (layer F.Cu) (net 3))
 (segment (start 156.991409 74.785001) (end 158.894999 74.785001) (width 0.25) (layer F.Cu) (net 3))
 (segment (start 156.59241 75.184) (end 156.991409 74.785001) (width 0.25) (layer F.Cu) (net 3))
 (segment (start 154.06061 76.44298) (end 155.32779 76.44298) (width 0.25) (layer F.Cu) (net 3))
 (segment (start 151.797001 77.564999) (end 152.938591 77.564999) (width 0.25) (layer F.Cu) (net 3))
 (segment (start 159.220001 74.459999) (end 160.02 73.66) (width 0.25) (layer F.Cu) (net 3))
 (segment (start 151.035001 78.326999) (end 151.797001 77.564999) (width 0.25) (layer F.Cu) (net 3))
 (segment (start 155.32779 76.44298) (end 156.58677 75.184) (width 0.25) (layer F.Cu) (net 3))
 (segment (start 152.938591 77.564999) (end 154.06061 76.44298) (width 0.25) (layer F.Cu) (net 3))
 (segment (start 151.035001 80.104999) (end 151.035001 78.326999) (width 0.25) (layer F.Cu) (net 3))
 (segment (start 149.86 81.28) (end 151.035001 80.104999) (width 0.25) (layer F.Cu) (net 3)))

